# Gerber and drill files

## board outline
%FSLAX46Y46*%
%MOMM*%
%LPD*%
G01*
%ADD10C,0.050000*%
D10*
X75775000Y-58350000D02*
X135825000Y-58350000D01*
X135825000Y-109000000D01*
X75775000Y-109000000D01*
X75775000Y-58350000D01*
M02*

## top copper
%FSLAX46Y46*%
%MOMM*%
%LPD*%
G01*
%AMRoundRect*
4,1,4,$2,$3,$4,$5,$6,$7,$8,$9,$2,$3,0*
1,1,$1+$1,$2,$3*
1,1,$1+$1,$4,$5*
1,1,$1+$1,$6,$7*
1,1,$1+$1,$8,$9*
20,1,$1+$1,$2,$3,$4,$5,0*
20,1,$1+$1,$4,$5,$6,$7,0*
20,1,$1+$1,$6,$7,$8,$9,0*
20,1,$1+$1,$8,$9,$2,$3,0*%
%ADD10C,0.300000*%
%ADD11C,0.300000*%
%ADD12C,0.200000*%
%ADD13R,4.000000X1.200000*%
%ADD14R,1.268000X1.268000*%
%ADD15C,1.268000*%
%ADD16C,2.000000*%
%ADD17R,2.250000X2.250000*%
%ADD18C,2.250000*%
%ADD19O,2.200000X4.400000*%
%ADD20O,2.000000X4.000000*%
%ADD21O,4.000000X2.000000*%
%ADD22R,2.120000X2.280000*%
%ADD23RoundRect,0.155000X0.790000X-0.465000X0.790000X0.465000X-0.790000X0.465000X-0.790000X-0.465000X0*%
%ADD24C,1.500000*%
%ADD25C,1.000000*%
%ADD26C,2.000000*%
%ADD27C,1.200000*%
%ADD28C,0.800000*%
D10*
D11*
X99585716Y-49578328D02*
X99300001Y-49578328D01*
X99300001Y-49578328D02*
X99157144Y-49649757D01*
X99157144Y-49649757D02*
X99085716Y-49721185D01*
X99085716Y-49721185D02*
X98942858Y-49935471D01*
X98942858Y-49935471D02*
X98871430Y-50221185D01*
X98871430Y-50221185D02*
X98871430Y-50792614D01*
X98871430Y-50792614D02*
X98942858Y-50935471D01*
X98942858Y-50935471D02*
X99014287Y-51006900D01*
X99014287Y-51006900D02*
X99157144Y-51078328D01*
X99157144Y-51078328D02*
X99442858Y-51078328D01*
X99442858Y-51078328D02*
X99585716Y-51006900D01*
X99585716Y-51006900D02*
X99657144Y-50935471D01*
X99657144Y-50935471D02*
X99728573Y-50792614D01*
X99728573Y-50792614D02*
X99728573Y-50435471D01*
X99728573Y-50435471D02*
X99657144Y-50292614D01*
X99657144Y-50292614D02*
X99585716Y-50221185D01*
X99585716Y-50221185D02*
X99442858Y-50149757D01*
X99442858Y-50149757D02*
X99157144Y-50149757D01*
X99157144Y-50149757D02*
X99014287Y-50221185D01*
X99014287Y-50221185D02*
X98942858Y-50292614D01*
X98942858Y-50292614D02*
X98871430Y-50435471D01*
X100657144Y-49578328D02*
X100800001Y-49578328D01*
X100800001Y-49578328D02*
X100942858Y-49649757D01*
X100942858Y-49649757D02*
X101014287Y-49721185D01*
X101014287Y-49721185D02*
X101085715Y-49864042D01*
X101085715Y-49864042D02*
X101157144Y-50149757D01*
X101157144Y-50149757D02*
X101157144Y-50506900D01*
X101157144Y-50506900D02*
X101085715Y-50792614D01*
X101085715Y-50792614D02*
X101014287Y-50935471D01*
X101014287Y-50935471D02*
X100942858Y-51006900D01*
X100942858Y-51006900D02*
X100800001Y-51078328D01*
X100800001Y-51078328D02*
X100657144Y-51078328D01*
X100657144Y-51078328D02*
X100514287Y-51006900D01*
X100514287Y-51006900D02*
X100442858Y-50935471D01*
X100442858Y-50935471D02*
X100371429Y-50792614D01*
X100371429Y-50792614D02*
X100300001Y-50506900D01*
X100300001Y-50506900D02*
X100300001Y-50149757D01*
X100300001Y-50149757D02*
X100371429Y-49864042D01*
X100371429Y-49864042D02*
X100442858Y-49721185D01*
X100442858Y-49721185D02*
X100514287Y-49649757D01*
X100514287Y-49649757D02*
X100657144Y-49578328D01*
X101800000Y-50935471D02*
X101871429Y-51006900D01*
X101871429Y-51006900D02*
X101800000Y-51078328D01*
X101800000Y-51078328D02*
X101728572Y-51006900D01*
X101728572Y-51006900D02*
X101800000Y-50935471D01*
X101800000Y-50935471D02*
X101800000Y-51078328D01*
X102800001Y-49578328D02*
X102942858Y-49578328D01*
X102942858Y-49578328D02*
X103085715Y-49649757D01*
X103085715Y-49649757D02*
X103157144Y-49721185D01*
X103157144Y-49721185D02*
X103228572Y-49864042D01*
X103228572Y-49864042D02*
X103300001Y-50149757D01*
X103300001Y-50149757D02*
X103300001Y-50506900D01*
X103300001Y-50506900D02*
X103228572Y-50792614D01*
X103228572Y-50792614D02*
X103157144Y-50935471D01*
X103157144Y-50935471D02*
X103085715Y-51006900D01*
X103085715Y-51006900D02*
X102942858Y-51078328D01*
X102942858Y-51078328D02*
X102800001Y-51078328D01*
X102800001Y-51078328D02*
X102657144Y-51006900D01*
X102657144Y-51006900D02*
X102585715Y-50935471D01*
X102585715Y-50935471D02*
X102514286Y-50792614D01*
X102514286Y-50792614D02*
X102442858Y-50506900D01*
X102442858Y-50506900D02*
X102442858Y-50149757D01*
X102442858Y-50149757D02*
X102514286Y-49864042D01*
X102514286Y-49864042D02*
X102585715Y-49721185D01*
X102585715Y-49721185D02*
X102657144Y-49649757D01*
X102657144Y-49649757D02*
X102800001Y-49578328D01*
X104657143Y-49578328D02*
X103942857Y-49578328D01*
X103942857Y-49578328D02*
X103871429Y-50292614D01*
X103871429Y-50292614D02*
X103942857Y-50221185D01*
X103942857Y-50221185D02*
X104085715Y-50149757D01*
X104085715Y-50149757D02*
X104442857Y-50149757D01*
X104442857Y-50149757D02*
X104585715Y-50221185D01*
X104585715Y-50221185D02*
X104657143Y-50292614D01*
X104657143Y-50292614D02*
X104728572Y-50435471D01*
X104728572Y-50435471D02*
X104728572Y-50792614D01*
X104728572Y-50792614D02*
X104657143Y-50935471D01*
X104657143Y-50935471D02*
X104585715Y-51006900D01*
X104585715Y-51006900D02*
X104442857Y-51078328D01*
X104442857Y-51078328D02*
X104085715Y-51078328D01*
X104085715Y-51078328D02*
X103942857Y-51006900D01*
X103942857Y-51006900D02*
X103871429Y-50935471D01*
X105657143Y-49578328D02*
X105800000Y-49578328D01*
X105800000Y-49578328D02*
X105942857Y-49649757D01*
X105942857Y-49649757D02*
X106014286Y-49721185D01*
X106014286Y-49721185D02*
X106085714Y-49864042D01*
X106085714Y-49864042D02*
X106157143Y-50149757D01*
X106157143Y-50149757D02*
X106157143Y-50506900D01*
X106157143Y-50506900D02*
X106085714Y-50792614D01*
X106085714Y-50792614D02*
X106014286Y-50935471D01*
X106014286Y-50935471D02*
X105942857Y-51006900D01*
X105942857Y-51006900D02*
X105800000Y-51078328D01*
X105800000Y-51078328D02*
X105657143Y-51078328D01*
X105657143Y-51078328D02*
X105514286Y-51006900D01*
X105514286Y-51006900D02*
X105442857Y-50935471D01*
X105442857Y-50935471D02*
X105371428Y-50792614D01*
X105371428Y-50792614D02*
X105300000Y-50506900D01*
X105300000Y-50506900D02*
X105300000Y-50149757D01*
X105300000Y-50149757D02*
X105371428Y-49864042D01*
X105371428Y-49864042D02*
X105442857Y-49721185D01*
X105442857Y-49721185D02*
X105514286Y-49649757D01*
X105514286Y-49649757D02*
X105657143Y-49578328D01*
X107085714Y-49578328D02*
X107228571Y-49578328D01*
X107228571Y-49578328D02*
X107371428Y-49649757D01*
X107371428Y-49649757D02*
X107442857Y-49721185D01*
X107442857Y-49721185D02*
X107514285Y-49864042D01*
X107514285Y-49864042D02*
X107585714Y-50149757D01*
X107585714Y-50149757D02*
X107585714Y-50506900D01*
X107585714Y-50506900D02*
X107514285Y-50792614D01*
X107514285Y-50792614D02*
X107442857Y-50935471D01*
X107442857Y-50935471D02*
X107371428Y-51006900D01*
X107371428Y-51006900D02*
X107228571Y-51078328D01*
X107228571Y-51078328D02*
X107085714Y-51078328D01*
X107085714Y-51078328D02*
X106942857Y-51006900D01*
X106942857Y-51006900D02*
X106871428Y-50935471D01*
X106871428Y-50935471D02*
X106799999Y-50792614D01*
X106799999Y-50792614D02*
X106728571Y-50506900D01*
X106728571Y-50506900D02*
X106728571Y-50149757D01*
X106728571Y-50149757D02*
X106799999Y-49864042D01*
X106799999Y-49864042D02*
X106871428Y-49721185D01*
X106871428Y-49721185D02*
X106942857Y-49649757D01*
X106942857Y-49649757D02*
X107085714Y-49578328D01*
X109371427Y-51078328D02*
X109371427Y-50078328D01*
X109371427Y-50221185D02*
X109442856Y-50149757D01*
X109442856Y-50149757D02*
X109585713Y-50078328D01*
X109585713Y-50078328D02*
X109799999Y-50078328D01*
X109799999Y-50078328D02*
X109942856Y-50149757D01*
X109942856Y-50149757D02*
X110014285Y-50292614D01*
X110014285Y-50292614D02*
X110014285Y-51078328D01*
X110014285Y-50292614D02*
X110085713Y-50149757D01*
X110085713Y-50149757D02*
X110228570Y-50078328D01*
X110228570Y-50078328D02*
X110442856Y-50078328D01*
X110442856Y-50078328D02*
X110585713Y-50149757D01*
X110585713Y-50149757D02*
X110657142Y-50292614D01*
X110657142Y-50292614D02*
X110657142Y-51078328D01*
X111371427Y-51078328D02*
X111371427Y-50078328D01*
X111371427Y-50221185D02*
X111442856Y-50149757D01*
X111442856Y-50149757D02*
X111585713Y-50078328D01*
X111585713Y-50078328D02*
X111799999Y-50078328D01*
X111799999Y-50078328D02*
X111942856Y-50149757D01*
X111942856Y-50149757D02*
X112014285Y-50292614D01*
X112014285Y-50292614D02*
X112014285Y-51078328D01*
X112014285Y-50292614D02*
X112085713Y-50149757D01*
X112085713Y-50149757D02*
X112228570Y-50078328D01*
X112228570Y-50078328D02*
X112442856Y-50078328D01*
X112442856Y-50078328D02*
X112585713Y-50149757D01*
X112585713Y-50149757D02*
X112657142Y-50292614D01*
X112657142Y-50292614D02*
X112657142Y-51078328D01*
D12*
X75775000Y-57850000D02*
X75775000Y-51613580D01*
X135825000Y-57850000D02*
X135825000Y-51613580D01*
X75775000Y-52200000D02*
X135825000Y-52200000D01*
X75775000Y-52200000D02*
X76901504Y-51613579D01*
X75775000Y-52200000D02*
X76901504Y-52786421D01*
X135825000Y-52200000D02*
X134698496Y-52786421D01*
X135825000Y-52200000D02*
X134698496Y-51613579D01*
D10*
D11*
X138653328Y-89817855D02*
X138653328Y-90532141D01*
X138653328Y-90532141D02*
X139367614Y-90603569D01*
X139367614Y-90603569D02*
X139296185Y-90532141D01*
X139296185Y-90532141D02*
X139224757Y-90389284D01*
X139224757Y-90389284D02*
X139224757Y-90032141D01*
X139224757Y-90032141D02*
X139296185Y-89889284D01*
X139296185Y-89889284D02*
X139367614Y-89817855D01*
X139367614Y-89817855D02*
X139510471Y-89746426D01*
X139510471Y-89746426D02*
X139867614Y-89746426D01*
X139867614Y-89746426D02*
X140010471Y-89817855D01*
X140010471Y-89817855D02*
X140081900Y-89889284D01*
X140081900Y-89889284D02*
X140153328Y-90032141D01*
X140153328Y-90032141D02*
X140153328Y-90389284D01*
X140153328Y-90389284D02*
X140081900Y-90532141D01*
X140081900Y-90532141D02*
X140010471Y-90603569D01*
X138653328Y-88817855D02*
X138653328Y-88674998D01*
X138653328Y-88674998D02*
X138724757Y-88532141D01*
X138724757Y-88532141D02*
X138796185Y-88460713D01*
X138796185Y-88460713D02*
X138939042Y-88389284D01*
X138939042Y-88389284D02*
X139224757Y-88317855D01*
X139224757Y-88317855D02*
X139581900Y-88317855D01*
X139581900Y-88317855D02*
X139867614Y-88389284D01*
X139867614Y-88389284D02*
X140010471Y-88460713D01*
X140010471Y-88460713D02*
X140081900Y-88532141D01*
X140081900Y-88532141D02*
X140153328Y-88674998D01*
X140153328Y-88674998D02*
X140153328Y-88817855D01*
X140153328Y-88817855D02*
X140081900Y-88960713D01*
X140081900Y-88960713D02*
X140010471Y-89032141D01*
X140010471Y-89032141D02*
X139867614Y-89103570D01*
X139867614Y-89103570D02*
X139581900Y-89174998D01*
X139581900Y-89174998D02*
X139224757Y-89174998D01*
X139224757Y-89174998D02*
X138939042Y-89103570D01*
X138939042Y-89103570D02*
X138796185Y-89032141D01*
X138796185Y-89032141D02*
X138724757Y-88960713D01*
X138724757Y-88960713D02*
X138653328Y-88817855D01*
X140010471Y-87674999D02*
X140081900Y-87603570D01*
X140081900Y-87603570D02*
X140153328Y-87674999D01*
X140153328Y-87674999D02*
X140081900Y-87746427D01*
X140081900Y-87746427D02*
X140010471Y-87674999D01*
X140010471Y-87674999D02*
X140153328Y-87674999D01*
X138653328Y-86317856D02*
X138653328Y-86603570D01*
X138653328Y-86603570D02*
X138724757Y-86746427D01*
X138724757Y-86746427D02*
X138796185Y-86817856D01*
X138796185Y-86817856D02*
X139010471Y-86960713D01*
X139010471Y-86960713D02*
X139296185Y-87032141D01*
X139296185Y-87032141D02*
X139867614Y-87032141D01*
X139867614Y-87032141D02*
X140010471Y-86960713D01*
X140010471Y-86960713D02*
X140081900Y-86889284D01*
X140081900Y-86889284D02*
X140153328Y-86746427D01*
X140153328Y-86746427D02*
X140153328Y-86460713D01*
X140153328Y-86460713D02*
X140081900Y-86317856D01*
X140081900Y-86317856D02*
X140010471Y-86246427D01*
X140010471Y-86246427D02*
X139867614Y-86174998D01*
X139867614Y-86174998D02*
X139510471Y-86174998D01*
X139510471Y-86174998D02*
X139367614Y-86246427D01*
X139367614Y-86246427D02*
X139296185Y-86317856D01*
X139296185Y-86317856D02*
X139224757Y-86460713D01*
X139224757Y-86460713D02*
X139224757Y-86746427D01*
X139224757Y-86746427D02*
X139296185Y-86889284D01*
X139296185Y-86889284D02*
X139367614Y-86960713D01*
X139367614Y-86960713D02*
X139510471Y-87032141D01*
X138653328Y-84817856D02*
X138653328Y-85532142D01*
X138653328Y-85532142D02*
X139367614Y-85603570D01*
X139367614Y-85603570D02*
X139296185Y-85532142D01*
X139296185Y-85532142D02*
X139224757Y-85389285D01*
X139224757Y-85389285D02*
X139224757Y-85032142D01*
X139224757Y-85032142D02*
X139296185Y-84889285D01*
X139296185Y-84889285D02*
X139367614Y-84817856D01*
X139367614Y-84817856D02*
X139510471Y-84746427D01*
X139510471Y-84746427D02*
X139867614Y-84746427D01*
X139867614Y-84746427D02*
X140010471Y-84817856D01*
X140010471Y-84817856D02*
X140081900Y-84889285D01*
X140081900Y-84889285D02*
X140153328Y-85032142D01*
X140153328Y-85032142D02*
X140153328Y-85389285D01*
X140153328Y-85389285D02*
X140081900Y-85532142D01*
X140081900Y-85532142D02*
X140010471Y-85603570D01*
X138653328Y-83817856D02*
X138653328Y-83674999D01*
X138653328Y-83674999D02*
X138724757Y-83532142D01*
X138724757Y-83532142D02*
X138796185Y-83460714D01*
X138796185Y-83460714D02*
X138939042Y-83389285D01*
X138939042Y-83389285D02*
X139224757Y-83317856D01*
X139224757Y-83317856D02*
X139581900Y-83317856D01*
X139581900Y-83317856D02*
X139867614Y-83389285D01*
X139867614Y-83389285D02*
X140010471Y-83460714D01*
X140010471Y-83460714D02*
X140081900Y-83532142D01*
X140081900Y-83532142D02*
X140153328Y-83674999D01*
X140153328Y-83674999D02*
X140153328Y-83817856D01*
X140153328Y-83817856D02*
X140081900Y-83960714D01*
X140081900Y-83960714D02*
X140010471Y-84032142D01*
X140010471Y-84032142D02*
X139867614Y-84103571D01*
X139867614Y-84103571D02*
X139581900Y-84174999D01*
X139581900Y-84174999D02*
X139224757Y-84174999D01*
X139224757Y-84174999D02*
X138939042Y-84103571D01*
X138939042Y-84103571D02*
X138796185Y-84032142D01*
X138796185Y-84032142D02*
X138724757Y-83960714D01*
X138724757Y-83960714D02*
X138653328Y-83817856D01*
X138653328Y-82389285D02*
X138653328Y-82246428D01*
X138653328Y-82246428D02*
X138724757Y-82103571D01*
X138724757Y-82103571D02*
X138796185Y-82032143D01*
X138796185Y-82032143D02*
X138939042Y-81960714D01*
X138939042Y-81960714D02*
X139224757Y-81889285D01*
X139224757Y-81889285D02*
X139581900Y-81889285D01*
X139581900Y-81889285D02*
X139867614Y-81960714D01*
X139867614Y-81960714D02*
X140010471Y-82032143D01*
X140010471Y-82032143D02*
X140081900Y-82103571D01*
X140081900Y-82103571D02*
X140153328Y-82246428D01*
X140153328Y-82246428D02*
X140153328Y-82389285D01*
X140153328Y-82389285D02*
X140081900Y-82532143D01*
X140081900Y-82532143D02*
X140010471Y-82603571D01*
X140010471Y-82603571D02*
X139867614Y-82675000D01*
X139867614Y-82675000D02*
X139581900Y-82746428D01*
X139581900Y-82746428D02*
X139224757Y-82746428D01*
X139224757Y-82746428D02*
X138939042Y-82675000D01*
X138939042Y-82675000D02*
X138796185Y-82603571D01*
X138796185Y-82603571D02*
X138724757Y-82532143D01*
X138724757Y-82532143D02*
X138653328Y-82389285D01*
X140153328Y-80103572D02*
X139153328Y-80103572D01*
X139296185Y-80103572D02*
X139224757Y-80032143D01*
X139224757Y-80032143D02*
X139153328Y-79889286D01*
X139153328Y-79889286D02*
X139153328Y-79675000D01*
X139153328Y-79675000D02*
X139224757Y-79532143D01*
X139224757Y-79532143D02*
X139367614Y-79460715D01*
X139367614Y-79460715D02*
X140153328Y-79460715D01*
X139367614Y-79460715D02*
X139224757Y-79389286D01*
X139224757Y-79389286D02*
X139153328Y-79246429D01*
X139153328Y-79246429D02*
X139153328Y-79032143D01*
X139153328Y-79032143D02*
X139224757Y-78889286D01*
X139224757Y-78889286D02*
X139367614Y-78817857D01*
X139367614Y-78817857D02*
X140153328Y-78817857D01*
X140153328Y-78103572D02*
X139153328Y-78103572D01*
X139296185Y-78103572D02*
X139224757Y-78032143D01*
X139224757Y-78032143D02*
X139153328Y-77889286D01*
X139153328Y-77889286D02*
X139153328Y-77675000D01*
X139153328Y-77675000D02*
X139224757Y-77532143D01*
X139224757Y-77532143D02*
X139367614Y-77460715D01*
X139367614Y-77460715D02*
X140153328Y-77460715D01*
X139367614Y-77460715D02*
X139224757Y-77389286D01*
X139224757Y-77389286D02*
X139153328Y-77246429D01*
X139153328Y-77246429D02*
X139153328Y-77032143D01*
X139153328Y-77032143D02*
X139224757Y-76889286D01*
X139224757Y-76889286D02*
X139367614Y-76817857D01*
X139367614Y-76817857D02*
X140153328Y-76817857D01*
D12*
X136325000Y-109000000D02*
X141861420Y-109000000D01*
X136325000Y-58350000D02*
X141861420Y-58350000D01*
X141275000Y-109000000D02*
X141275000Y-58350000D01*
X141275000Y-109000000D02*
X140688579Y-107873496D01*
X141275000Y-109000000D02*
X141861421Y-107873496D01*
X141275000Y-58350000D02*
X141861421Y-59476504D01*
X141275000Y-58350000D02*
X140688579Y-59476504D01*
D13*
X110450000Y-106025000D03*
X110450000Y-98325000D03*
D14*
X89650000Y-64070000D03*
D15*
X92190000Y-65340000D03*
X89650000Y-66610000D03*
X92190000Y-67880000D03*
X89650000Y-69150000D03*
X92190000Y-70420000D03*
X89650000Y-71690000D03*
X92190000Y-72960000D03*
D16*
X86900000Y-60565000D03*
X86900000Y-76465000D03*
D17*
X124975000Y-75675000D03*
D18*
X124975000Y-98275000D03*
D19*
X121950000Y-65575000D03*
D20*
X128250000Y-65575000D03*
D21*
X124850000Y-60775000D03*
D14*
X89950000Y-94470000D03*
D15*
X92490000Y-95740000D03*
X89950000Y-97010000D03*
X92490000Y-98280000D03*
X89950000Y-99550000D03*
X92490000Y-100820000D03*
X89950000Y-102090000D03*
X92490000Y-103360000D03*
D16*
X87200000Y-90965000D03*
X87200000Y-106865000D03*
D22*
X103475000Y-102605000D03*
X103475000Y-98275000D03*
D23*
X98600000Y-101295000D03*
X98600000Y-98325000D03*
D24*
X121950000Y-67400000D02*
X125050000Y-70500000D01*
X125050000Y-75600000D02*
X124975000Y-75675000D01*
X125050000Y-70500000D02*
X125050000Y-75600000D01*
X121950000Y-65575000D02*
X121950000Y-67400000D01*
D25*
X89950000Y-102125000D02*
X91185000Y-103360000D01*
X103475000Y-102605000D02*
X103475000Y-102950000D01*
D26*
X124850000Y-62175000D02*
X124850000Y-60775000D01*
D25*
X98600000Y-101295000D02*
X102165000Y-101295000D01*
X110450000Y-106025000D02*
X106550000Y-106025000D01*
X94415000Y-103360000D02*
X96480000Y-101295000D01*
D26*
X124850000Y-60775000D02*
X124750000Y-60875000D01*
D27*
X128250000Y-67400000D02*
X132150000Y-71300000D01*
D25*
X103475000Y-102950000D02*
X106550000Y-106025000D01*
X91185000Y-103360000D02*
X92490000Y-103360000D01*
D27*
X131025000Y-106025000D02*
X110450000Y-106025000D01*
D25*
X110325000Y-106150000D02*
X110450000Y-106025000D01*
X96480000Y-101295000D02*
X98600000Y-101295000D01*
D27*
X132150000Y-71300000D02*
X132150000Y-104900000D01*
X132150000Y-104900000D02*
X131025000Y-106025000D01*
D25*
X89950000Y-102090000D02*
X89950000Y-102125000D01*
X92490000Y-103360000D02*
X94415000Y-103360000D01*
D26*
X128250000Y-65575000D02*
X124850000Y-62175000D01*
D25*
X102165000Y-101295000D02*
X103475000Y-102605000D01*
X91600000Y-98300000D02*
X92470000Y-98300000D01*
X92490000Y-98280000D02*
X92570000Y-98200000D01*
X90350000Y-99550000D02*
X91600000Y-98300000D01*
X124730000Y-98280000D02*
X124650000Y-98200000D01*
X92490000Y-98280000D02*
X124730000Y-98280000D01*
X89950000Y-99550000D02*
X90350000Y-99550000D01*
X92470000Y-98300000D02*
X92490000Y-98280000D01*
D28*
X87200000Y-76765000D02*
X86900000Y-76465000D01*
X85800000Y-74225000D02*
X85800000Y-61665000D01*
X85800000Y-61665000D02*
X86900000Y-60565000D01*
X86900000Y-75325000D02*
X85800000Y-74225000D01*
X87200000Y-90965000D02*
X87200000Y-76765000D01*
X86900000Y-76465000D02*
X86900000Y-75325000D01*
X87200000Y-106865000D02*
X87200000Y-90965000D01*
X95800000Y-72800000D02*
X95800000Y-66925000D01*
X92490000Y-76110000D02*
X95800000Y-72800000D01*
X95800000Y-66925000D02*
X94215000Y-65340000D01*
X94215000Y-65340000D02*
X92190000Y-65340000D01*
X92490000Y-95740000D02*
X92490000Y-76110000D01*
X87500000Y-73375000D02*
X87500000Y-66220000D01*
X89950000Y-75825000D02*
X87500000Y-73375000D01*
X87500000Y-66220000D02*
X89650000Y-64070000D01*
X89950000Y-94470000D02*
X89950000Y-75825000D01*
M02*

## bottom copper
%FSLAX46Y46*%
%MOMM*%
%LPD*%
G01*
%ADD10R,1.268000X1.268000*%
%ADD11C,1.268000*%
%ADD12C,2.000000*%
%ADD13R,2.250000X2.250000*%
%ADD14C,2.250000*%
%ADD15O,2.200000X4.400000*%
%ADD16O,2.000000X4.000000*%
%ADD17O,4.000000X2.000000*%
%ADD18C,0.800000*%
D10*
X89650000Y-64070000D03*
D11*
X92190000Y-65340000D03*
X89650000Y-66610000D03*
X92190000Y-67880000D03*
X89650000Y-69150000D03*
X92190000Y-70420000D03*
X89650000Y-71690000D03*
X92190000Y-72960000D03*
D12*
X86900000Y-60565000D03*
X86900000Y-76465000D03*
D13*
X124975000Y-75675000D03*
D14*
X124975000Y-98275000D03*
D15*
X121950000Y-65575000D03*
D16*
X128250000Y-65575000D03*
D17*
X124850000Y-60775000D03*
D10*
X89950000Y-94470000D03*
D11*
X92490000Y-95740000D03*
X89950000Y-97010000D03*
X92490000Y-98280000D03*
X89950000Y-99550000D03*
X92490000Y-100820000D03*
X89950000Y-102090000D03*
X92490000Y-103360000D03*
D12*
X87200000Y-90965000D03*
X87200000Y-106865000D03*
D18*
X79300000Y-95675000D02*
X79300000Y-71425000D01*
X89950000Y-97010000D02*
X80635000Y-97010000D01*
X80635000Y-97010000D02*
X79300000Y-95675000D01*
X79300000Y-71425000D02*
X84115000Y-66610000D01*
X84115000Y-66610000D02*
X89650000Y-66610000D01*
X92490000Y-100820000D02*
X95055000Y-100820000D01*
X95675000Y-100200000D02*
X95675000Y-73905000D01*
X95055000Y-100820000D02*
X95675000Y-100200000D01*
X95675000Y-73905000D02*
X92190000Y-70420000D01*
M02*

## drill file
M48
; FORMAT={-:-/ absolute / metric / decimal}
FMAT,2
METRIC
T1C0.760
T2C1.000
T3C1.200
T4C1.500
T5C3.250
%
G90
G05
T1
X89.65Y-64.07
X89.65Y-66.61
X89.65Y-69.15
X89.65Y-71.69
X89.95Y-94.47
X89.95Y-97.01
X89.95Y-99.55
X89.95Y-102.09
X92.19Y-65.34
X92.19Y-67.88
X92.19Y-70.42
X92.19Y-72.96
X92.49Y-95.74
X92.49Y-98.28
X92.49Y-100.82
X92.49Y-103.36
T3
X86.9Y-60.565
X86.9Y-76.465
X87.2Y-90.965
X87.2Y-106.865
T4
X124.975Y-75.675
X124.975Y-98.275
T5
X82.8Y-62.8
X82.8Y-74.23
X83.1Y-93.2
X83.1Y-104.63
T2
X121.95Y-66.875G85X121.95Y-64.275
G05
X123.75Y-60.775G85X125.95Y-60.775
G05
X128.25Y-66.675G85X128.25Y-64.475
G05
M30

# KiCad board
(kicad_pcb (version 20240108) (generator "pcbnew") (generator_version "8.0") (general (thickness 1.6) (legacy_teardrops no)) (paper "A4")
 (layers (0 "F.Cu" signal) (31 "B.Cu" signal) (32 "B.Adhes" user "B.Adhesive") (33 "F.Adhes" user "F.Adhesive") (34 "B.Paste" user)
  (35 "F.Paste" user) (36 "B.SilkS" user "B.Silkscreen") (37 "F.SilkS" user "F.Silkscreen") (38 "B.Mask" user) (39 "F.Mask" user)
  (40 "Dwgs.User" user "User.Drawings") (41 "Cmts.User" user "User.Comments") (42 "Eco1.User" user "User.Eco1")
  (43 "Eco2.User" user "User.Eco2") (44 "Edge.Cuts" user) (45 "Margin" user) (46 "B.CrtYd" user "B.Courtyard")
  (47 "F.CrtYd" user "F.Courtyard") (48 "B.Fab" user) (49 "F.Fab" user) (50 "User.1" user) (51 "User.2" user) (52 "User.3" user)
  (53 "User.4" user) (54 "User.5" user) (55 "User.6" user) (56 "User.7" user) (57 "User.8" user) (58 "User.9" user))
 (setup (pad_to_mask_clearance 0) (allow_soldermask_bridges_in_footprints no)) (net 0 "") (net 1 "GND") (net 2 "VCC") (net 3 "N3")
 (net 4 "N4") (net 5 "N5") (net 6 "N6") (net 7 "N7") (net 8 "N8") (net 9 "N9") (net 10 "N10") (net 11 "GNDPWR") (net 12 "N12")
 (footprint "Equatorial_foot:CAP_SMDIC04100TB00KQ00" (layer "F.Cu") (at 110.45 102.175 90)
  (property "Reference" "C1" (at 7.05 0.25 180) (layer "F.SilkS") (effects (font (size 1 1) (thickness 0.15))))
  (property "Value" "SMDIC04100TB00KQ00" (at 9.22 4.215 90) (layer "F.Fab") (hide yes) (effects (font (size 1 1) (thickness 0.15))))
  (pad "1" smd rect (at -3.85 0 90) (size 1.2 4) (layers "F.Cu" "F.Paste" "F.Mask") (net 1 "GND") (solder_mask_margin 0.102))
  (pad "2" smd rect (at 3.85 0 90) (size 1.2 4) (layers "F.Cu" "F.Paste" "F.Mask") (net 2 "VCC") (solder_mask_margin 0.102)))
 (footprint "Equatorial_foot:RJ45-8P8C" (layer "F.Cu") (at 83.3 68.515 -90)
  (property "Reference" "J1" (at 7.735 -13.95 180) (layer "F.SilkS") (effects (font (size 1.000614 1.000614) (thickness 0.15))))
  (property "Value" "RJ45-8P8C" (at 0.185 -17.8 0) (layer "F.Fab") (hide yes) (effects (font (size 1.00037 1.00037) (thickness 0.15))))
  (pad "" np_thru_hole circle (at -5.715 0.5 270) (size 3.25 3.25) (drill 3.25) (layers "*.Cu" "*.Mask"))
  (pad "" np_thru_hole circle (at 5.715 0.5 270) (size 3.25 3.25) (drill 3.25) (layers "*.Cu" "*.Mask"))
  (pad "1" thru_hole rect (at -4.445 -6.35 270) (size 1.268 1.268) (drill 0.76) (layers "*.Cu" "*.Mask") (remove_unused_layers no)
   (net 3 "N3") (solder_mask_margin 0.102))
  (pad "2" thru_hole circle (at -3.175 -8.89 270) (size 1.268 1.268) (drill 0.76) (layers "*.Cu" "*.Mask") (remove_unused_layers no)
   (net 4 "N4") (solder_mask_margin 0.102))
  (pad "3" thru_hole circle (at -1.905 -6.35 270) (size 1.268 1.268) (drill 0.76) (layers "*.Cu" "*.Mask") (remove_unused_layers no)
   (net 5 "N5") (solder_mask_margin 0.102))
  (pad "4" thru_hole circle (at -0.635 -8.89 270) (size 1.268 1.268) (drill 0.76) (layers "*.Cu" "*.Mask") (remove_unused_layers no)
   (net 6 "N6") (solder_mask_margin 0.102))
  (pad "5" thru_hole circle (at 0.635 -6.35 270) (size 1.268 1.268) (drill 0.76) (layers "*.Cu" "*.Mask") (remove_unused_layers no)
   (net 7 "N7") (solder_mask_margin 0.102))
  (pad "6" thru_hole circle (at 1.905 -8.89 270) (size 1.268 1.268) (drill 0.76) (layers "*.Cu" "*.Mask") (remove_unused_layers no)
   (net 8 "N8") (solder_mask_margin 0.102))
  (pad "7" thru_hole circle (at 3.175 -6.35 270) (size 1.268 1.268) (drill 0.76) (layers "*.Cu" "*.Mask") (remove_unused_layers no)
   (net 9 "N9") (solder_mask_margin 0.102))
  (pad "8" thru_hole circle (at 4.445 -8.89 270) (size 1.268 1.268) (drill 0.76) (layers "*.Cu" "*.Mask") (remove_unused_layers no)
   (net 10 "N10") (solder_mask_margin 0.102))
  (pad "9" thru_hole circle (at -7.95 -3.6 270) (size 2 2) (drill 1.2) (layers "*.Cu" "*.Mask") (remove_unused_layers no) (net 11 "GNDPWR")
   (solder_mask_margin 0.102))
  (pad "10" thru_hole circle (at 7.95 -3.6 270) (size 2 2) (drill 1.2) (layers "*.Cu" "*.Mask") (remove_unused_layers no) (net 11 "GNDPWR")
   (solder_mask_margin 0.102)))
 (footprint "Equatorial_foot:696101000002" (layer "F.Cu") (at 124.975 75.675 -90)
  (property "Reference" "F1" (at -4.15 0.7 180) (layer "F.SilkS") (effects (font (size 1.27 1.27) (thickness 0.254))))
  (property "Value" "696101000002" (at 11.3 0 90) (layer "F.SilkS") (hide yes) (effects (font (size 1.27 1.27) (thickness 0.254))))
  (pad "1" thru_hole rect (at 0 0 270) (size 2.25 2.25) (drill 1.5) (layers "*.Cu" "*.Mask") (remove_unused_layers no) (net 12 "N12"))
  (pad "2" thru_hole circle (at 22.6 0 270) (size 2.25 2.25) (drill 1.5) (layers "*.Cu" "*.Mask") (remove_unused_layers no) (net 2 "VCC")))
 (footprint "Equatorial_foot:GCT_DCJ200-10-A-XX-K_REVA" (layer "F.Cu") (at 128.5 65.575 90)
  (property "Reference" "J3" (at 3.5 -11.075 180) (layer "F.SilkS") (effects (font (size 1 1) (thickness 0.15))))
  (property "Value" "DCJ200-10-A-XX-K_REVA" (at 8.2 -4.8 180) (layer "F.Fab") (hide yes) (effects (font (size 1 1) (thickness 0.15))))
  (pad "1" thru_hole oval (at 0 -6.55 90) (size 4.4 2.2) (drill oval 3.6 1) (layers "*.Cu" "*.Mask") (remove_unused_layers no)
   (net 12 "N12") (solder_mask_margin 0.102))
  (pad "2" thru_hole oval (at 0 -0.25 90) (size 4 2) (drill oval 3.2 1) (layers "*.Cu" "*.Mask") (remove_unused_layers no) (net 1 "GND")
   (solder_mask_margin 0.102))
  (pad "3" thru_hole oval (at 4.8 -3.65 90) (size 2 4) (drill oval 1 3.2) (layers "*.Cu" "*.Mask") (remove_unused_layers no) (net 1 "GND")
   (solder_mask_margin 0.102)))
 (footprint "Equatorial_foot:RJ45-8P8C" (layer "F.Cu") (at 83.6 98.915 -90)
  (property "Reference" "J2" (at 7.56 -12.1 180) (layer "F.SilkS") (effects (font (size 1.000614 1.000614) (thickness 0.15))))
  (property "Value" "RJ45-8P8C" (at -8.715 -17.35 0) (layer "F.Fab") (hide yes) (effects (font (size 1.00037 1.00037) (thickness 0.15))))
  (pad "" np_thru_hole circle (at -5.715 0.5 270) (size 3.25 3.25) (drill 3.25) (layers "*.Cu" "*.Mask"))
  (pad "" np_thru_hole circle (at 5.715 0.5 270) (size 3.25 3.25) (drill 3.25) (layers "*.Cu" "*.Mask"))
  (pad "1" thru_hole rect (at -4.445 -6.35 270) (size 1.268 1.268) (drill 0.76) (layers "*.Cu" "*.Mask") (remove_unused_layers no)
   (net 3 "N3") (solder_mask_margin 0.102))
  (pad "2" thru_hole circle (at -3.175 -8.89 270) (size 1.268 1.268) (drill 0.76) (layers "*.Cu" "*.Mask") (remove_unused_layers no)
   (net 4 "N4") (solder_mask_margin 0.102))
  (pad "3" thru_hole circle (at -1.905 -6.35 270) (size 1.268 1.268) (drill 0.76) (layers "*.Cu" "*.Mask") (remove_unused_layers no)
   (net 5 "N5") (solder_mask_margin 0.102))
  (pad "4" thru_hole circle (at -0.635 -8.89 270) (size 1.268 1.268) (drill 0.76) (layers "*.Cu" "*.Mask") (remove_unused_layers no)
   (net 2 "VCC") (solder_mask_margin 0.102))
  (pad "5" thru_hole circle (at 0.635 -6.35 270) (size 1.268 1.268) (drill 0.76) (layers "*.Cu" "*.Mask") (remove_unused_layers no)
   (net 2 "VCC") (solder_mask_margin 0.102))
  (pad "6" thru_hole circle (at 1.905 -8.89 270) (size 1.268 1.268) (drill 0.76) (layers "*.Cu" "*.Mask") (remove_unused_layers no)
   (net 8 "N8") (solder_mask_margin 0.102))
  (pad "7" thru_hole circle (at 3.175 -6.35 270) (size 1.268 1.268) (drill 0.76) (layers "*.Cu" "*.Mask") (remove_unused_layers no)
   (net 1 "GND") (solder_mask_margin 0.102))
  (pad "8" thru_hole circle (at 4.445 -8.89 270) (size 1.268 1.268) (drill 0.76) (layers "*.Cu" "*.Mask") (remove_unused_layers no)
   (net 1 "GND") (solder_mask_margin 0.102))
  (pad "9" thru_hole circle (at -7.95 -3.6 270) (size 2 2) (drill 1.2) (layers "*.Cu" "*.Mask") (remove_unused_layers no) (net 11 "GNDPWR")
   (solder_mask_margin 0.102))
  (pad "10" thru_hole circle (at 7.95 -3.6 270) (size 2 2) (drill 1.2) (layers "*.Cu" "*.Mask") (remove_unused_layers no) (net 11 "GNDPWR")
   (solder_mask_margin 0.102)))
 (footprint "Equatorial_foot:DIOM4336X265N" (layer "F.Cu") (at 103.475 100.44 -90)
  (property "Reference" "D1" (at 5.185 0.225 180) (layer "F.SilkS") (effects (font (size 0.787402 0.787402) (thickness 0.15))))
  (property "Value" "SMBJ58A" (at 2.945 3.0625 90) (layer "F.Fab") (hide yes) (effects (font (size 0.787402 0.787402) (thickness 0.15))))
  (pad "A" smd rect (at 2.165 0 270) (size 2.28 2.12) (layers "F.Cu" "F.Paste" "F.Mask") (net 1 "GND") (solder_mask_margin 0.102))
  (pad "C" smd rect (at -2.165 0 270) (size 2.28 2.12) (layers "F.Cu" "F.Paste" "F.Mask") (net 2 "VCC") (solder_mask_margin 0.102)))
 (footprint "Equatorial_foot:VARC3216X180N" (layer "F.Cu") (at 98.6 99.81 90)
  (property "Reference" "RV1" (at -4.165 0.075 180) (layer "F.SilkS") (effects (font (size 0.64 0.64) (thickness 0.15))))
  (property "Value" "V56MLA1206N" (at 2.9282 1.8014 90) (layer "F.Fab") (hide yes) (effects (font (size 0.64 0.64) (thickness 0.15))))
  (pad "1" smd roundrect (at -1.485 0 90) (size 1.24 1.89) (layers "F.Cu" "F.Paste" "F.Mask") (roundrect_rratio 0.125) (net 1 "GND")
   (solder_mask_margin 0.102))
  (pad "2" smd roundrect (at 1.485 0 90) (size 1.24 1.89) (layers "F.Cu" "F.Paste" "F.Mask") (roundrect_rratio 0.125) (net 2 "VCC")
   (solder_mask_margin 0.102)))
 (gr_rect (start 75.775 58.35) (end 135.825 109) (stroke (width 0.05) (type default)) (fill none) (layer "Edge.Cuts"))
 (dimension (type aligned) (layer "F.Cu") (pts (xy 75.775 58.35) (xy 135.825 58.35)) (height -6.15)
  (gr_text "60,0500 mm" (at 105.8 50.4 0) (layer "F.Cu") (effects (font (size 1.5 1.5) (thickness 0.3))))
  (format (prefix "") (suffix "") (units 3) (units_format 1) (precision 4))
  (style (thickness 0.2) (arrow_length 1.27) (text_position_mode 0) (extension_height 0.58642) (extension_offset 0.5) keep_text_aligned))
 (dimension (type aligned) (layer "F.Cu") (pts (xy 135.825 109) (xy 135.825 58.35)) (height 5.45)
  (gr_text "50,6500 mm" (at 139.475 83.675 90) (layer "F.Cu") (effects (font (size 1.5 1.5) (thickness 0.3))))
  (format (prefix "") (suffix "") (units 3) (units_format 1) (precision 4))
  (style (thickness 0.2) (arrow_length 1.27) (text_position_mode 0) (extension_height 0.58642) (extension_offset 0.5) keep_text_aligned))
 (segment (start 121.95 67.4) (end 125.05 70.5) (width 1.5) (layer "F.Cu") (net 12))
 (segment (start 125.05 75.6) (end 124.975 75.675) (width 1.5) (layer "F.Cu") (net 12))
 (segment (start 125.05 70.5) (end 125.05 75.6) (width 1.5) (layer "F.Cu") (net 12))
 (segment (start 121.95 65.575) (end 121.95 67.4) (width 1.5) (layer "F.Cu") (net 12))
 (segment (start 89.95 102.125) (end 91.185 103.36) (width 1) (layer "F.Cu") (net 1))
 (segment (start 103.475 102.605) (end 103.475 102.95) (width 1) (layer "F.Cu") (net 1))
 (segment (start 124.85 62.175) (end 124.85 60.775) (width 2) (layer "F.Cu") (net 1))
 (segment (start 98.6 101.295) (end 102.165 101.295) (width 1) (layer "F.Cu") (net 1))
 (segment (start 110.45 106.025) (end 106.55 106.025) (width 1) (layer "F.Cu") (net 1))
 (segment (start 94.415 103.36) (end 96.48 101.295) (width 1) (layer "F.Cu") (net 1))
 (segment (start 124.85 60.775) (end 124.75 60.875) (width 2) (layer "F.Cu") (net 1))
 (segment (start 128.25 67.4) (end 132.15 71.3) (width 1.2) (layer "F.Cu") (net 1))
 (segment (start 103.475 102.95) (end 106.55 106.025) (width 1) (layer "F.Cu") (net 1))
 (segment (start 91.185 103.36) (end 92.49 103.36) (width 1) (layer "F.Cu") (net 1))
 (segment (start 131.025 106.025) (end 110.45 106.025) (width 1.2) (layer "F.Cu") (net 1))
 (segment (start 110.325 106.15) (end 110.45 106.025) (width 1) (layer "F.Cu") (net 1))
 (segment (start 96.48 101.295) (end 98.6 101.295) (width 1) (layer "F.Cu") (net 1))
 (segment (start 132.15 71.3) (end 132.15 104.9) (width 1.2) (layer "F.Cu") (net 1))
 (segment (start 132.15 104.9) (end 131.025 106.025) (width 1.2) (layer "F.Cu") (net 1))
 (segment (start 89.95 102.09) (end 89.95 102.125) (width 1) (layer "F.Cu") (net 1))
 (segment (start 92.49 103.36) (end 94.415 103.36) (width 1) (layer "F.Cu") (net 1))
 (segment (start 128.25 65.575) (end 124.85 62.175) (width 2) (layer "F.Cu") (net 1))
 (segment (start 102.165 101.295) (end 103.475 102.605) (width 1) (layer "F.Cu") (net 1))
 (segment (start 91.6 98.3) (end 92.47 98.3) (width 1) (layer "F.Cu") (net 2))
 (segment (start 92.49 98.28) (end 92.57 98.2) (width 1) (layer "F.Cu") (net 2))
 (segment (start 90.35 99.55) (end 91.6 98.3) (width 1) (layer "F.Cu") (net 2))
 (segment (start 124.73 98.28) (end 124.65 98.2) (width 1) (layer "F.Cu") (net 2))
 (segment (start 92.49 98.28) (end 124.73 98.28) (width 1) (layer "F.Cu") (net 2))
 (segment (start 89.95 99.55) (end 90.35 99.55) (width 1) (layer "F.Cu") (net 2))
 (segment (start 92.47 98.3) (end 92.49 98.28) (width 1) (layer "F.Cu") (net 2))
 (segment (start 87.2 76.765) (end 86.9 76.465) (width 0.8) (layer "F.Cu") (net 11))
 (segment (start 85.8 74.225) (end 85.8 61.665) (width 0.8) (layer "F.Cu") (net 11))
 (segment (start 85.8 61.665) (end 86.9 60.565) (width 0.8) (layer "F.Cu") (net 11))
 (segment (start 86.9 75.325) (end 85.8 74.225) (width 0.8) (layer "F.Cu") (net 11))
 (segment (start 87.2 90.965) (end 87.2 76.765) (width 0.8) (layer "F.Cu") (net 11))
 (segment (start 86.9 76.465) (end 86.9 75.325) (width 0.8) (layer "F.Cu") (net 11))
 (segment (start 87.2 106.865) (end 87.2 90.965) (width 0.8) (layer "F.Cu") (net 11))
 (segment (start 95.8 72.8) (end 95.8 66.925) (width 0.8) (layer "F.Cu") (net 4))
 (segment (start 92.49 76.11) (end 95.8 72.8) (width 0.8) (layer "F.Cu") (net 4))
 (segment (start 95.8 66.925) (end 94.215 65.34) (width 0.8) (layer "F.Cu") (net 4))
 (segment (start 94.215 65.34) (end 92.19 65.34) (width 0.8) (layer "F.Cu") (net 4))
 (segment (start 92.49 95.74) (end 92.49 76.11) (width 0.8) (layer "F.Cu") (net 4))
 (segment (start 79.3 95.675) (end 79.3 71.425) (width 0.8) (layer "B.Cu") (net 5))
 (segment (start 89.95 97.01) (end 80.635 97.01) (width 0.8) (layer "B.Cu") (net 5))
 (segment (start 80.635 97.01) (end 79.3 95.675) (width 0.8) (layer "B.Cu") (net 5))
 (segment (start 79.3 71.425) (end 84.115 66.61) (width 0.8) (layer "B.Cu") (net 5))
 (segment (start 84.115 66.61) (end 89.65 66.61) (width 0.8) (layer "B.Cu") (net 5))
 (segment (start 92.49 100.82) (end 95.055 100.82) (width 0.8) (layer "B.Cu") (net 8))
 (segment (start 95.675 100.2) (end 95.675 73.905) (width 0.8) (layer "B.Cu") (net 8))
 (segment (start 95.055 100.82) (end 95.675 100.2) (width 0.8) (layer "B.Cu") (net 8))
 (segment (start 95.675 73.905) (end 92.19 70.42) (width 0.8) (layer "B.Cu") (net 8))
 (segment (start 87.5 73.375) (end 87.5 66.22) (width 0.8) (layer "F.Cu") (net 3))
 (segment (start 89.95 75.825) (end 87.5 73.375) (width 0.8) (layer "F.Cu") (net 3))
 (segment (start 87.5 66.22) (end 89.65 64.07) (width 0.8) (layer "F.Cu") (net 3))
 (segment (start 89.95 94.47) (end 89.95 75.825) (width 0.8) (layer "F.Cu") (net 3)))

